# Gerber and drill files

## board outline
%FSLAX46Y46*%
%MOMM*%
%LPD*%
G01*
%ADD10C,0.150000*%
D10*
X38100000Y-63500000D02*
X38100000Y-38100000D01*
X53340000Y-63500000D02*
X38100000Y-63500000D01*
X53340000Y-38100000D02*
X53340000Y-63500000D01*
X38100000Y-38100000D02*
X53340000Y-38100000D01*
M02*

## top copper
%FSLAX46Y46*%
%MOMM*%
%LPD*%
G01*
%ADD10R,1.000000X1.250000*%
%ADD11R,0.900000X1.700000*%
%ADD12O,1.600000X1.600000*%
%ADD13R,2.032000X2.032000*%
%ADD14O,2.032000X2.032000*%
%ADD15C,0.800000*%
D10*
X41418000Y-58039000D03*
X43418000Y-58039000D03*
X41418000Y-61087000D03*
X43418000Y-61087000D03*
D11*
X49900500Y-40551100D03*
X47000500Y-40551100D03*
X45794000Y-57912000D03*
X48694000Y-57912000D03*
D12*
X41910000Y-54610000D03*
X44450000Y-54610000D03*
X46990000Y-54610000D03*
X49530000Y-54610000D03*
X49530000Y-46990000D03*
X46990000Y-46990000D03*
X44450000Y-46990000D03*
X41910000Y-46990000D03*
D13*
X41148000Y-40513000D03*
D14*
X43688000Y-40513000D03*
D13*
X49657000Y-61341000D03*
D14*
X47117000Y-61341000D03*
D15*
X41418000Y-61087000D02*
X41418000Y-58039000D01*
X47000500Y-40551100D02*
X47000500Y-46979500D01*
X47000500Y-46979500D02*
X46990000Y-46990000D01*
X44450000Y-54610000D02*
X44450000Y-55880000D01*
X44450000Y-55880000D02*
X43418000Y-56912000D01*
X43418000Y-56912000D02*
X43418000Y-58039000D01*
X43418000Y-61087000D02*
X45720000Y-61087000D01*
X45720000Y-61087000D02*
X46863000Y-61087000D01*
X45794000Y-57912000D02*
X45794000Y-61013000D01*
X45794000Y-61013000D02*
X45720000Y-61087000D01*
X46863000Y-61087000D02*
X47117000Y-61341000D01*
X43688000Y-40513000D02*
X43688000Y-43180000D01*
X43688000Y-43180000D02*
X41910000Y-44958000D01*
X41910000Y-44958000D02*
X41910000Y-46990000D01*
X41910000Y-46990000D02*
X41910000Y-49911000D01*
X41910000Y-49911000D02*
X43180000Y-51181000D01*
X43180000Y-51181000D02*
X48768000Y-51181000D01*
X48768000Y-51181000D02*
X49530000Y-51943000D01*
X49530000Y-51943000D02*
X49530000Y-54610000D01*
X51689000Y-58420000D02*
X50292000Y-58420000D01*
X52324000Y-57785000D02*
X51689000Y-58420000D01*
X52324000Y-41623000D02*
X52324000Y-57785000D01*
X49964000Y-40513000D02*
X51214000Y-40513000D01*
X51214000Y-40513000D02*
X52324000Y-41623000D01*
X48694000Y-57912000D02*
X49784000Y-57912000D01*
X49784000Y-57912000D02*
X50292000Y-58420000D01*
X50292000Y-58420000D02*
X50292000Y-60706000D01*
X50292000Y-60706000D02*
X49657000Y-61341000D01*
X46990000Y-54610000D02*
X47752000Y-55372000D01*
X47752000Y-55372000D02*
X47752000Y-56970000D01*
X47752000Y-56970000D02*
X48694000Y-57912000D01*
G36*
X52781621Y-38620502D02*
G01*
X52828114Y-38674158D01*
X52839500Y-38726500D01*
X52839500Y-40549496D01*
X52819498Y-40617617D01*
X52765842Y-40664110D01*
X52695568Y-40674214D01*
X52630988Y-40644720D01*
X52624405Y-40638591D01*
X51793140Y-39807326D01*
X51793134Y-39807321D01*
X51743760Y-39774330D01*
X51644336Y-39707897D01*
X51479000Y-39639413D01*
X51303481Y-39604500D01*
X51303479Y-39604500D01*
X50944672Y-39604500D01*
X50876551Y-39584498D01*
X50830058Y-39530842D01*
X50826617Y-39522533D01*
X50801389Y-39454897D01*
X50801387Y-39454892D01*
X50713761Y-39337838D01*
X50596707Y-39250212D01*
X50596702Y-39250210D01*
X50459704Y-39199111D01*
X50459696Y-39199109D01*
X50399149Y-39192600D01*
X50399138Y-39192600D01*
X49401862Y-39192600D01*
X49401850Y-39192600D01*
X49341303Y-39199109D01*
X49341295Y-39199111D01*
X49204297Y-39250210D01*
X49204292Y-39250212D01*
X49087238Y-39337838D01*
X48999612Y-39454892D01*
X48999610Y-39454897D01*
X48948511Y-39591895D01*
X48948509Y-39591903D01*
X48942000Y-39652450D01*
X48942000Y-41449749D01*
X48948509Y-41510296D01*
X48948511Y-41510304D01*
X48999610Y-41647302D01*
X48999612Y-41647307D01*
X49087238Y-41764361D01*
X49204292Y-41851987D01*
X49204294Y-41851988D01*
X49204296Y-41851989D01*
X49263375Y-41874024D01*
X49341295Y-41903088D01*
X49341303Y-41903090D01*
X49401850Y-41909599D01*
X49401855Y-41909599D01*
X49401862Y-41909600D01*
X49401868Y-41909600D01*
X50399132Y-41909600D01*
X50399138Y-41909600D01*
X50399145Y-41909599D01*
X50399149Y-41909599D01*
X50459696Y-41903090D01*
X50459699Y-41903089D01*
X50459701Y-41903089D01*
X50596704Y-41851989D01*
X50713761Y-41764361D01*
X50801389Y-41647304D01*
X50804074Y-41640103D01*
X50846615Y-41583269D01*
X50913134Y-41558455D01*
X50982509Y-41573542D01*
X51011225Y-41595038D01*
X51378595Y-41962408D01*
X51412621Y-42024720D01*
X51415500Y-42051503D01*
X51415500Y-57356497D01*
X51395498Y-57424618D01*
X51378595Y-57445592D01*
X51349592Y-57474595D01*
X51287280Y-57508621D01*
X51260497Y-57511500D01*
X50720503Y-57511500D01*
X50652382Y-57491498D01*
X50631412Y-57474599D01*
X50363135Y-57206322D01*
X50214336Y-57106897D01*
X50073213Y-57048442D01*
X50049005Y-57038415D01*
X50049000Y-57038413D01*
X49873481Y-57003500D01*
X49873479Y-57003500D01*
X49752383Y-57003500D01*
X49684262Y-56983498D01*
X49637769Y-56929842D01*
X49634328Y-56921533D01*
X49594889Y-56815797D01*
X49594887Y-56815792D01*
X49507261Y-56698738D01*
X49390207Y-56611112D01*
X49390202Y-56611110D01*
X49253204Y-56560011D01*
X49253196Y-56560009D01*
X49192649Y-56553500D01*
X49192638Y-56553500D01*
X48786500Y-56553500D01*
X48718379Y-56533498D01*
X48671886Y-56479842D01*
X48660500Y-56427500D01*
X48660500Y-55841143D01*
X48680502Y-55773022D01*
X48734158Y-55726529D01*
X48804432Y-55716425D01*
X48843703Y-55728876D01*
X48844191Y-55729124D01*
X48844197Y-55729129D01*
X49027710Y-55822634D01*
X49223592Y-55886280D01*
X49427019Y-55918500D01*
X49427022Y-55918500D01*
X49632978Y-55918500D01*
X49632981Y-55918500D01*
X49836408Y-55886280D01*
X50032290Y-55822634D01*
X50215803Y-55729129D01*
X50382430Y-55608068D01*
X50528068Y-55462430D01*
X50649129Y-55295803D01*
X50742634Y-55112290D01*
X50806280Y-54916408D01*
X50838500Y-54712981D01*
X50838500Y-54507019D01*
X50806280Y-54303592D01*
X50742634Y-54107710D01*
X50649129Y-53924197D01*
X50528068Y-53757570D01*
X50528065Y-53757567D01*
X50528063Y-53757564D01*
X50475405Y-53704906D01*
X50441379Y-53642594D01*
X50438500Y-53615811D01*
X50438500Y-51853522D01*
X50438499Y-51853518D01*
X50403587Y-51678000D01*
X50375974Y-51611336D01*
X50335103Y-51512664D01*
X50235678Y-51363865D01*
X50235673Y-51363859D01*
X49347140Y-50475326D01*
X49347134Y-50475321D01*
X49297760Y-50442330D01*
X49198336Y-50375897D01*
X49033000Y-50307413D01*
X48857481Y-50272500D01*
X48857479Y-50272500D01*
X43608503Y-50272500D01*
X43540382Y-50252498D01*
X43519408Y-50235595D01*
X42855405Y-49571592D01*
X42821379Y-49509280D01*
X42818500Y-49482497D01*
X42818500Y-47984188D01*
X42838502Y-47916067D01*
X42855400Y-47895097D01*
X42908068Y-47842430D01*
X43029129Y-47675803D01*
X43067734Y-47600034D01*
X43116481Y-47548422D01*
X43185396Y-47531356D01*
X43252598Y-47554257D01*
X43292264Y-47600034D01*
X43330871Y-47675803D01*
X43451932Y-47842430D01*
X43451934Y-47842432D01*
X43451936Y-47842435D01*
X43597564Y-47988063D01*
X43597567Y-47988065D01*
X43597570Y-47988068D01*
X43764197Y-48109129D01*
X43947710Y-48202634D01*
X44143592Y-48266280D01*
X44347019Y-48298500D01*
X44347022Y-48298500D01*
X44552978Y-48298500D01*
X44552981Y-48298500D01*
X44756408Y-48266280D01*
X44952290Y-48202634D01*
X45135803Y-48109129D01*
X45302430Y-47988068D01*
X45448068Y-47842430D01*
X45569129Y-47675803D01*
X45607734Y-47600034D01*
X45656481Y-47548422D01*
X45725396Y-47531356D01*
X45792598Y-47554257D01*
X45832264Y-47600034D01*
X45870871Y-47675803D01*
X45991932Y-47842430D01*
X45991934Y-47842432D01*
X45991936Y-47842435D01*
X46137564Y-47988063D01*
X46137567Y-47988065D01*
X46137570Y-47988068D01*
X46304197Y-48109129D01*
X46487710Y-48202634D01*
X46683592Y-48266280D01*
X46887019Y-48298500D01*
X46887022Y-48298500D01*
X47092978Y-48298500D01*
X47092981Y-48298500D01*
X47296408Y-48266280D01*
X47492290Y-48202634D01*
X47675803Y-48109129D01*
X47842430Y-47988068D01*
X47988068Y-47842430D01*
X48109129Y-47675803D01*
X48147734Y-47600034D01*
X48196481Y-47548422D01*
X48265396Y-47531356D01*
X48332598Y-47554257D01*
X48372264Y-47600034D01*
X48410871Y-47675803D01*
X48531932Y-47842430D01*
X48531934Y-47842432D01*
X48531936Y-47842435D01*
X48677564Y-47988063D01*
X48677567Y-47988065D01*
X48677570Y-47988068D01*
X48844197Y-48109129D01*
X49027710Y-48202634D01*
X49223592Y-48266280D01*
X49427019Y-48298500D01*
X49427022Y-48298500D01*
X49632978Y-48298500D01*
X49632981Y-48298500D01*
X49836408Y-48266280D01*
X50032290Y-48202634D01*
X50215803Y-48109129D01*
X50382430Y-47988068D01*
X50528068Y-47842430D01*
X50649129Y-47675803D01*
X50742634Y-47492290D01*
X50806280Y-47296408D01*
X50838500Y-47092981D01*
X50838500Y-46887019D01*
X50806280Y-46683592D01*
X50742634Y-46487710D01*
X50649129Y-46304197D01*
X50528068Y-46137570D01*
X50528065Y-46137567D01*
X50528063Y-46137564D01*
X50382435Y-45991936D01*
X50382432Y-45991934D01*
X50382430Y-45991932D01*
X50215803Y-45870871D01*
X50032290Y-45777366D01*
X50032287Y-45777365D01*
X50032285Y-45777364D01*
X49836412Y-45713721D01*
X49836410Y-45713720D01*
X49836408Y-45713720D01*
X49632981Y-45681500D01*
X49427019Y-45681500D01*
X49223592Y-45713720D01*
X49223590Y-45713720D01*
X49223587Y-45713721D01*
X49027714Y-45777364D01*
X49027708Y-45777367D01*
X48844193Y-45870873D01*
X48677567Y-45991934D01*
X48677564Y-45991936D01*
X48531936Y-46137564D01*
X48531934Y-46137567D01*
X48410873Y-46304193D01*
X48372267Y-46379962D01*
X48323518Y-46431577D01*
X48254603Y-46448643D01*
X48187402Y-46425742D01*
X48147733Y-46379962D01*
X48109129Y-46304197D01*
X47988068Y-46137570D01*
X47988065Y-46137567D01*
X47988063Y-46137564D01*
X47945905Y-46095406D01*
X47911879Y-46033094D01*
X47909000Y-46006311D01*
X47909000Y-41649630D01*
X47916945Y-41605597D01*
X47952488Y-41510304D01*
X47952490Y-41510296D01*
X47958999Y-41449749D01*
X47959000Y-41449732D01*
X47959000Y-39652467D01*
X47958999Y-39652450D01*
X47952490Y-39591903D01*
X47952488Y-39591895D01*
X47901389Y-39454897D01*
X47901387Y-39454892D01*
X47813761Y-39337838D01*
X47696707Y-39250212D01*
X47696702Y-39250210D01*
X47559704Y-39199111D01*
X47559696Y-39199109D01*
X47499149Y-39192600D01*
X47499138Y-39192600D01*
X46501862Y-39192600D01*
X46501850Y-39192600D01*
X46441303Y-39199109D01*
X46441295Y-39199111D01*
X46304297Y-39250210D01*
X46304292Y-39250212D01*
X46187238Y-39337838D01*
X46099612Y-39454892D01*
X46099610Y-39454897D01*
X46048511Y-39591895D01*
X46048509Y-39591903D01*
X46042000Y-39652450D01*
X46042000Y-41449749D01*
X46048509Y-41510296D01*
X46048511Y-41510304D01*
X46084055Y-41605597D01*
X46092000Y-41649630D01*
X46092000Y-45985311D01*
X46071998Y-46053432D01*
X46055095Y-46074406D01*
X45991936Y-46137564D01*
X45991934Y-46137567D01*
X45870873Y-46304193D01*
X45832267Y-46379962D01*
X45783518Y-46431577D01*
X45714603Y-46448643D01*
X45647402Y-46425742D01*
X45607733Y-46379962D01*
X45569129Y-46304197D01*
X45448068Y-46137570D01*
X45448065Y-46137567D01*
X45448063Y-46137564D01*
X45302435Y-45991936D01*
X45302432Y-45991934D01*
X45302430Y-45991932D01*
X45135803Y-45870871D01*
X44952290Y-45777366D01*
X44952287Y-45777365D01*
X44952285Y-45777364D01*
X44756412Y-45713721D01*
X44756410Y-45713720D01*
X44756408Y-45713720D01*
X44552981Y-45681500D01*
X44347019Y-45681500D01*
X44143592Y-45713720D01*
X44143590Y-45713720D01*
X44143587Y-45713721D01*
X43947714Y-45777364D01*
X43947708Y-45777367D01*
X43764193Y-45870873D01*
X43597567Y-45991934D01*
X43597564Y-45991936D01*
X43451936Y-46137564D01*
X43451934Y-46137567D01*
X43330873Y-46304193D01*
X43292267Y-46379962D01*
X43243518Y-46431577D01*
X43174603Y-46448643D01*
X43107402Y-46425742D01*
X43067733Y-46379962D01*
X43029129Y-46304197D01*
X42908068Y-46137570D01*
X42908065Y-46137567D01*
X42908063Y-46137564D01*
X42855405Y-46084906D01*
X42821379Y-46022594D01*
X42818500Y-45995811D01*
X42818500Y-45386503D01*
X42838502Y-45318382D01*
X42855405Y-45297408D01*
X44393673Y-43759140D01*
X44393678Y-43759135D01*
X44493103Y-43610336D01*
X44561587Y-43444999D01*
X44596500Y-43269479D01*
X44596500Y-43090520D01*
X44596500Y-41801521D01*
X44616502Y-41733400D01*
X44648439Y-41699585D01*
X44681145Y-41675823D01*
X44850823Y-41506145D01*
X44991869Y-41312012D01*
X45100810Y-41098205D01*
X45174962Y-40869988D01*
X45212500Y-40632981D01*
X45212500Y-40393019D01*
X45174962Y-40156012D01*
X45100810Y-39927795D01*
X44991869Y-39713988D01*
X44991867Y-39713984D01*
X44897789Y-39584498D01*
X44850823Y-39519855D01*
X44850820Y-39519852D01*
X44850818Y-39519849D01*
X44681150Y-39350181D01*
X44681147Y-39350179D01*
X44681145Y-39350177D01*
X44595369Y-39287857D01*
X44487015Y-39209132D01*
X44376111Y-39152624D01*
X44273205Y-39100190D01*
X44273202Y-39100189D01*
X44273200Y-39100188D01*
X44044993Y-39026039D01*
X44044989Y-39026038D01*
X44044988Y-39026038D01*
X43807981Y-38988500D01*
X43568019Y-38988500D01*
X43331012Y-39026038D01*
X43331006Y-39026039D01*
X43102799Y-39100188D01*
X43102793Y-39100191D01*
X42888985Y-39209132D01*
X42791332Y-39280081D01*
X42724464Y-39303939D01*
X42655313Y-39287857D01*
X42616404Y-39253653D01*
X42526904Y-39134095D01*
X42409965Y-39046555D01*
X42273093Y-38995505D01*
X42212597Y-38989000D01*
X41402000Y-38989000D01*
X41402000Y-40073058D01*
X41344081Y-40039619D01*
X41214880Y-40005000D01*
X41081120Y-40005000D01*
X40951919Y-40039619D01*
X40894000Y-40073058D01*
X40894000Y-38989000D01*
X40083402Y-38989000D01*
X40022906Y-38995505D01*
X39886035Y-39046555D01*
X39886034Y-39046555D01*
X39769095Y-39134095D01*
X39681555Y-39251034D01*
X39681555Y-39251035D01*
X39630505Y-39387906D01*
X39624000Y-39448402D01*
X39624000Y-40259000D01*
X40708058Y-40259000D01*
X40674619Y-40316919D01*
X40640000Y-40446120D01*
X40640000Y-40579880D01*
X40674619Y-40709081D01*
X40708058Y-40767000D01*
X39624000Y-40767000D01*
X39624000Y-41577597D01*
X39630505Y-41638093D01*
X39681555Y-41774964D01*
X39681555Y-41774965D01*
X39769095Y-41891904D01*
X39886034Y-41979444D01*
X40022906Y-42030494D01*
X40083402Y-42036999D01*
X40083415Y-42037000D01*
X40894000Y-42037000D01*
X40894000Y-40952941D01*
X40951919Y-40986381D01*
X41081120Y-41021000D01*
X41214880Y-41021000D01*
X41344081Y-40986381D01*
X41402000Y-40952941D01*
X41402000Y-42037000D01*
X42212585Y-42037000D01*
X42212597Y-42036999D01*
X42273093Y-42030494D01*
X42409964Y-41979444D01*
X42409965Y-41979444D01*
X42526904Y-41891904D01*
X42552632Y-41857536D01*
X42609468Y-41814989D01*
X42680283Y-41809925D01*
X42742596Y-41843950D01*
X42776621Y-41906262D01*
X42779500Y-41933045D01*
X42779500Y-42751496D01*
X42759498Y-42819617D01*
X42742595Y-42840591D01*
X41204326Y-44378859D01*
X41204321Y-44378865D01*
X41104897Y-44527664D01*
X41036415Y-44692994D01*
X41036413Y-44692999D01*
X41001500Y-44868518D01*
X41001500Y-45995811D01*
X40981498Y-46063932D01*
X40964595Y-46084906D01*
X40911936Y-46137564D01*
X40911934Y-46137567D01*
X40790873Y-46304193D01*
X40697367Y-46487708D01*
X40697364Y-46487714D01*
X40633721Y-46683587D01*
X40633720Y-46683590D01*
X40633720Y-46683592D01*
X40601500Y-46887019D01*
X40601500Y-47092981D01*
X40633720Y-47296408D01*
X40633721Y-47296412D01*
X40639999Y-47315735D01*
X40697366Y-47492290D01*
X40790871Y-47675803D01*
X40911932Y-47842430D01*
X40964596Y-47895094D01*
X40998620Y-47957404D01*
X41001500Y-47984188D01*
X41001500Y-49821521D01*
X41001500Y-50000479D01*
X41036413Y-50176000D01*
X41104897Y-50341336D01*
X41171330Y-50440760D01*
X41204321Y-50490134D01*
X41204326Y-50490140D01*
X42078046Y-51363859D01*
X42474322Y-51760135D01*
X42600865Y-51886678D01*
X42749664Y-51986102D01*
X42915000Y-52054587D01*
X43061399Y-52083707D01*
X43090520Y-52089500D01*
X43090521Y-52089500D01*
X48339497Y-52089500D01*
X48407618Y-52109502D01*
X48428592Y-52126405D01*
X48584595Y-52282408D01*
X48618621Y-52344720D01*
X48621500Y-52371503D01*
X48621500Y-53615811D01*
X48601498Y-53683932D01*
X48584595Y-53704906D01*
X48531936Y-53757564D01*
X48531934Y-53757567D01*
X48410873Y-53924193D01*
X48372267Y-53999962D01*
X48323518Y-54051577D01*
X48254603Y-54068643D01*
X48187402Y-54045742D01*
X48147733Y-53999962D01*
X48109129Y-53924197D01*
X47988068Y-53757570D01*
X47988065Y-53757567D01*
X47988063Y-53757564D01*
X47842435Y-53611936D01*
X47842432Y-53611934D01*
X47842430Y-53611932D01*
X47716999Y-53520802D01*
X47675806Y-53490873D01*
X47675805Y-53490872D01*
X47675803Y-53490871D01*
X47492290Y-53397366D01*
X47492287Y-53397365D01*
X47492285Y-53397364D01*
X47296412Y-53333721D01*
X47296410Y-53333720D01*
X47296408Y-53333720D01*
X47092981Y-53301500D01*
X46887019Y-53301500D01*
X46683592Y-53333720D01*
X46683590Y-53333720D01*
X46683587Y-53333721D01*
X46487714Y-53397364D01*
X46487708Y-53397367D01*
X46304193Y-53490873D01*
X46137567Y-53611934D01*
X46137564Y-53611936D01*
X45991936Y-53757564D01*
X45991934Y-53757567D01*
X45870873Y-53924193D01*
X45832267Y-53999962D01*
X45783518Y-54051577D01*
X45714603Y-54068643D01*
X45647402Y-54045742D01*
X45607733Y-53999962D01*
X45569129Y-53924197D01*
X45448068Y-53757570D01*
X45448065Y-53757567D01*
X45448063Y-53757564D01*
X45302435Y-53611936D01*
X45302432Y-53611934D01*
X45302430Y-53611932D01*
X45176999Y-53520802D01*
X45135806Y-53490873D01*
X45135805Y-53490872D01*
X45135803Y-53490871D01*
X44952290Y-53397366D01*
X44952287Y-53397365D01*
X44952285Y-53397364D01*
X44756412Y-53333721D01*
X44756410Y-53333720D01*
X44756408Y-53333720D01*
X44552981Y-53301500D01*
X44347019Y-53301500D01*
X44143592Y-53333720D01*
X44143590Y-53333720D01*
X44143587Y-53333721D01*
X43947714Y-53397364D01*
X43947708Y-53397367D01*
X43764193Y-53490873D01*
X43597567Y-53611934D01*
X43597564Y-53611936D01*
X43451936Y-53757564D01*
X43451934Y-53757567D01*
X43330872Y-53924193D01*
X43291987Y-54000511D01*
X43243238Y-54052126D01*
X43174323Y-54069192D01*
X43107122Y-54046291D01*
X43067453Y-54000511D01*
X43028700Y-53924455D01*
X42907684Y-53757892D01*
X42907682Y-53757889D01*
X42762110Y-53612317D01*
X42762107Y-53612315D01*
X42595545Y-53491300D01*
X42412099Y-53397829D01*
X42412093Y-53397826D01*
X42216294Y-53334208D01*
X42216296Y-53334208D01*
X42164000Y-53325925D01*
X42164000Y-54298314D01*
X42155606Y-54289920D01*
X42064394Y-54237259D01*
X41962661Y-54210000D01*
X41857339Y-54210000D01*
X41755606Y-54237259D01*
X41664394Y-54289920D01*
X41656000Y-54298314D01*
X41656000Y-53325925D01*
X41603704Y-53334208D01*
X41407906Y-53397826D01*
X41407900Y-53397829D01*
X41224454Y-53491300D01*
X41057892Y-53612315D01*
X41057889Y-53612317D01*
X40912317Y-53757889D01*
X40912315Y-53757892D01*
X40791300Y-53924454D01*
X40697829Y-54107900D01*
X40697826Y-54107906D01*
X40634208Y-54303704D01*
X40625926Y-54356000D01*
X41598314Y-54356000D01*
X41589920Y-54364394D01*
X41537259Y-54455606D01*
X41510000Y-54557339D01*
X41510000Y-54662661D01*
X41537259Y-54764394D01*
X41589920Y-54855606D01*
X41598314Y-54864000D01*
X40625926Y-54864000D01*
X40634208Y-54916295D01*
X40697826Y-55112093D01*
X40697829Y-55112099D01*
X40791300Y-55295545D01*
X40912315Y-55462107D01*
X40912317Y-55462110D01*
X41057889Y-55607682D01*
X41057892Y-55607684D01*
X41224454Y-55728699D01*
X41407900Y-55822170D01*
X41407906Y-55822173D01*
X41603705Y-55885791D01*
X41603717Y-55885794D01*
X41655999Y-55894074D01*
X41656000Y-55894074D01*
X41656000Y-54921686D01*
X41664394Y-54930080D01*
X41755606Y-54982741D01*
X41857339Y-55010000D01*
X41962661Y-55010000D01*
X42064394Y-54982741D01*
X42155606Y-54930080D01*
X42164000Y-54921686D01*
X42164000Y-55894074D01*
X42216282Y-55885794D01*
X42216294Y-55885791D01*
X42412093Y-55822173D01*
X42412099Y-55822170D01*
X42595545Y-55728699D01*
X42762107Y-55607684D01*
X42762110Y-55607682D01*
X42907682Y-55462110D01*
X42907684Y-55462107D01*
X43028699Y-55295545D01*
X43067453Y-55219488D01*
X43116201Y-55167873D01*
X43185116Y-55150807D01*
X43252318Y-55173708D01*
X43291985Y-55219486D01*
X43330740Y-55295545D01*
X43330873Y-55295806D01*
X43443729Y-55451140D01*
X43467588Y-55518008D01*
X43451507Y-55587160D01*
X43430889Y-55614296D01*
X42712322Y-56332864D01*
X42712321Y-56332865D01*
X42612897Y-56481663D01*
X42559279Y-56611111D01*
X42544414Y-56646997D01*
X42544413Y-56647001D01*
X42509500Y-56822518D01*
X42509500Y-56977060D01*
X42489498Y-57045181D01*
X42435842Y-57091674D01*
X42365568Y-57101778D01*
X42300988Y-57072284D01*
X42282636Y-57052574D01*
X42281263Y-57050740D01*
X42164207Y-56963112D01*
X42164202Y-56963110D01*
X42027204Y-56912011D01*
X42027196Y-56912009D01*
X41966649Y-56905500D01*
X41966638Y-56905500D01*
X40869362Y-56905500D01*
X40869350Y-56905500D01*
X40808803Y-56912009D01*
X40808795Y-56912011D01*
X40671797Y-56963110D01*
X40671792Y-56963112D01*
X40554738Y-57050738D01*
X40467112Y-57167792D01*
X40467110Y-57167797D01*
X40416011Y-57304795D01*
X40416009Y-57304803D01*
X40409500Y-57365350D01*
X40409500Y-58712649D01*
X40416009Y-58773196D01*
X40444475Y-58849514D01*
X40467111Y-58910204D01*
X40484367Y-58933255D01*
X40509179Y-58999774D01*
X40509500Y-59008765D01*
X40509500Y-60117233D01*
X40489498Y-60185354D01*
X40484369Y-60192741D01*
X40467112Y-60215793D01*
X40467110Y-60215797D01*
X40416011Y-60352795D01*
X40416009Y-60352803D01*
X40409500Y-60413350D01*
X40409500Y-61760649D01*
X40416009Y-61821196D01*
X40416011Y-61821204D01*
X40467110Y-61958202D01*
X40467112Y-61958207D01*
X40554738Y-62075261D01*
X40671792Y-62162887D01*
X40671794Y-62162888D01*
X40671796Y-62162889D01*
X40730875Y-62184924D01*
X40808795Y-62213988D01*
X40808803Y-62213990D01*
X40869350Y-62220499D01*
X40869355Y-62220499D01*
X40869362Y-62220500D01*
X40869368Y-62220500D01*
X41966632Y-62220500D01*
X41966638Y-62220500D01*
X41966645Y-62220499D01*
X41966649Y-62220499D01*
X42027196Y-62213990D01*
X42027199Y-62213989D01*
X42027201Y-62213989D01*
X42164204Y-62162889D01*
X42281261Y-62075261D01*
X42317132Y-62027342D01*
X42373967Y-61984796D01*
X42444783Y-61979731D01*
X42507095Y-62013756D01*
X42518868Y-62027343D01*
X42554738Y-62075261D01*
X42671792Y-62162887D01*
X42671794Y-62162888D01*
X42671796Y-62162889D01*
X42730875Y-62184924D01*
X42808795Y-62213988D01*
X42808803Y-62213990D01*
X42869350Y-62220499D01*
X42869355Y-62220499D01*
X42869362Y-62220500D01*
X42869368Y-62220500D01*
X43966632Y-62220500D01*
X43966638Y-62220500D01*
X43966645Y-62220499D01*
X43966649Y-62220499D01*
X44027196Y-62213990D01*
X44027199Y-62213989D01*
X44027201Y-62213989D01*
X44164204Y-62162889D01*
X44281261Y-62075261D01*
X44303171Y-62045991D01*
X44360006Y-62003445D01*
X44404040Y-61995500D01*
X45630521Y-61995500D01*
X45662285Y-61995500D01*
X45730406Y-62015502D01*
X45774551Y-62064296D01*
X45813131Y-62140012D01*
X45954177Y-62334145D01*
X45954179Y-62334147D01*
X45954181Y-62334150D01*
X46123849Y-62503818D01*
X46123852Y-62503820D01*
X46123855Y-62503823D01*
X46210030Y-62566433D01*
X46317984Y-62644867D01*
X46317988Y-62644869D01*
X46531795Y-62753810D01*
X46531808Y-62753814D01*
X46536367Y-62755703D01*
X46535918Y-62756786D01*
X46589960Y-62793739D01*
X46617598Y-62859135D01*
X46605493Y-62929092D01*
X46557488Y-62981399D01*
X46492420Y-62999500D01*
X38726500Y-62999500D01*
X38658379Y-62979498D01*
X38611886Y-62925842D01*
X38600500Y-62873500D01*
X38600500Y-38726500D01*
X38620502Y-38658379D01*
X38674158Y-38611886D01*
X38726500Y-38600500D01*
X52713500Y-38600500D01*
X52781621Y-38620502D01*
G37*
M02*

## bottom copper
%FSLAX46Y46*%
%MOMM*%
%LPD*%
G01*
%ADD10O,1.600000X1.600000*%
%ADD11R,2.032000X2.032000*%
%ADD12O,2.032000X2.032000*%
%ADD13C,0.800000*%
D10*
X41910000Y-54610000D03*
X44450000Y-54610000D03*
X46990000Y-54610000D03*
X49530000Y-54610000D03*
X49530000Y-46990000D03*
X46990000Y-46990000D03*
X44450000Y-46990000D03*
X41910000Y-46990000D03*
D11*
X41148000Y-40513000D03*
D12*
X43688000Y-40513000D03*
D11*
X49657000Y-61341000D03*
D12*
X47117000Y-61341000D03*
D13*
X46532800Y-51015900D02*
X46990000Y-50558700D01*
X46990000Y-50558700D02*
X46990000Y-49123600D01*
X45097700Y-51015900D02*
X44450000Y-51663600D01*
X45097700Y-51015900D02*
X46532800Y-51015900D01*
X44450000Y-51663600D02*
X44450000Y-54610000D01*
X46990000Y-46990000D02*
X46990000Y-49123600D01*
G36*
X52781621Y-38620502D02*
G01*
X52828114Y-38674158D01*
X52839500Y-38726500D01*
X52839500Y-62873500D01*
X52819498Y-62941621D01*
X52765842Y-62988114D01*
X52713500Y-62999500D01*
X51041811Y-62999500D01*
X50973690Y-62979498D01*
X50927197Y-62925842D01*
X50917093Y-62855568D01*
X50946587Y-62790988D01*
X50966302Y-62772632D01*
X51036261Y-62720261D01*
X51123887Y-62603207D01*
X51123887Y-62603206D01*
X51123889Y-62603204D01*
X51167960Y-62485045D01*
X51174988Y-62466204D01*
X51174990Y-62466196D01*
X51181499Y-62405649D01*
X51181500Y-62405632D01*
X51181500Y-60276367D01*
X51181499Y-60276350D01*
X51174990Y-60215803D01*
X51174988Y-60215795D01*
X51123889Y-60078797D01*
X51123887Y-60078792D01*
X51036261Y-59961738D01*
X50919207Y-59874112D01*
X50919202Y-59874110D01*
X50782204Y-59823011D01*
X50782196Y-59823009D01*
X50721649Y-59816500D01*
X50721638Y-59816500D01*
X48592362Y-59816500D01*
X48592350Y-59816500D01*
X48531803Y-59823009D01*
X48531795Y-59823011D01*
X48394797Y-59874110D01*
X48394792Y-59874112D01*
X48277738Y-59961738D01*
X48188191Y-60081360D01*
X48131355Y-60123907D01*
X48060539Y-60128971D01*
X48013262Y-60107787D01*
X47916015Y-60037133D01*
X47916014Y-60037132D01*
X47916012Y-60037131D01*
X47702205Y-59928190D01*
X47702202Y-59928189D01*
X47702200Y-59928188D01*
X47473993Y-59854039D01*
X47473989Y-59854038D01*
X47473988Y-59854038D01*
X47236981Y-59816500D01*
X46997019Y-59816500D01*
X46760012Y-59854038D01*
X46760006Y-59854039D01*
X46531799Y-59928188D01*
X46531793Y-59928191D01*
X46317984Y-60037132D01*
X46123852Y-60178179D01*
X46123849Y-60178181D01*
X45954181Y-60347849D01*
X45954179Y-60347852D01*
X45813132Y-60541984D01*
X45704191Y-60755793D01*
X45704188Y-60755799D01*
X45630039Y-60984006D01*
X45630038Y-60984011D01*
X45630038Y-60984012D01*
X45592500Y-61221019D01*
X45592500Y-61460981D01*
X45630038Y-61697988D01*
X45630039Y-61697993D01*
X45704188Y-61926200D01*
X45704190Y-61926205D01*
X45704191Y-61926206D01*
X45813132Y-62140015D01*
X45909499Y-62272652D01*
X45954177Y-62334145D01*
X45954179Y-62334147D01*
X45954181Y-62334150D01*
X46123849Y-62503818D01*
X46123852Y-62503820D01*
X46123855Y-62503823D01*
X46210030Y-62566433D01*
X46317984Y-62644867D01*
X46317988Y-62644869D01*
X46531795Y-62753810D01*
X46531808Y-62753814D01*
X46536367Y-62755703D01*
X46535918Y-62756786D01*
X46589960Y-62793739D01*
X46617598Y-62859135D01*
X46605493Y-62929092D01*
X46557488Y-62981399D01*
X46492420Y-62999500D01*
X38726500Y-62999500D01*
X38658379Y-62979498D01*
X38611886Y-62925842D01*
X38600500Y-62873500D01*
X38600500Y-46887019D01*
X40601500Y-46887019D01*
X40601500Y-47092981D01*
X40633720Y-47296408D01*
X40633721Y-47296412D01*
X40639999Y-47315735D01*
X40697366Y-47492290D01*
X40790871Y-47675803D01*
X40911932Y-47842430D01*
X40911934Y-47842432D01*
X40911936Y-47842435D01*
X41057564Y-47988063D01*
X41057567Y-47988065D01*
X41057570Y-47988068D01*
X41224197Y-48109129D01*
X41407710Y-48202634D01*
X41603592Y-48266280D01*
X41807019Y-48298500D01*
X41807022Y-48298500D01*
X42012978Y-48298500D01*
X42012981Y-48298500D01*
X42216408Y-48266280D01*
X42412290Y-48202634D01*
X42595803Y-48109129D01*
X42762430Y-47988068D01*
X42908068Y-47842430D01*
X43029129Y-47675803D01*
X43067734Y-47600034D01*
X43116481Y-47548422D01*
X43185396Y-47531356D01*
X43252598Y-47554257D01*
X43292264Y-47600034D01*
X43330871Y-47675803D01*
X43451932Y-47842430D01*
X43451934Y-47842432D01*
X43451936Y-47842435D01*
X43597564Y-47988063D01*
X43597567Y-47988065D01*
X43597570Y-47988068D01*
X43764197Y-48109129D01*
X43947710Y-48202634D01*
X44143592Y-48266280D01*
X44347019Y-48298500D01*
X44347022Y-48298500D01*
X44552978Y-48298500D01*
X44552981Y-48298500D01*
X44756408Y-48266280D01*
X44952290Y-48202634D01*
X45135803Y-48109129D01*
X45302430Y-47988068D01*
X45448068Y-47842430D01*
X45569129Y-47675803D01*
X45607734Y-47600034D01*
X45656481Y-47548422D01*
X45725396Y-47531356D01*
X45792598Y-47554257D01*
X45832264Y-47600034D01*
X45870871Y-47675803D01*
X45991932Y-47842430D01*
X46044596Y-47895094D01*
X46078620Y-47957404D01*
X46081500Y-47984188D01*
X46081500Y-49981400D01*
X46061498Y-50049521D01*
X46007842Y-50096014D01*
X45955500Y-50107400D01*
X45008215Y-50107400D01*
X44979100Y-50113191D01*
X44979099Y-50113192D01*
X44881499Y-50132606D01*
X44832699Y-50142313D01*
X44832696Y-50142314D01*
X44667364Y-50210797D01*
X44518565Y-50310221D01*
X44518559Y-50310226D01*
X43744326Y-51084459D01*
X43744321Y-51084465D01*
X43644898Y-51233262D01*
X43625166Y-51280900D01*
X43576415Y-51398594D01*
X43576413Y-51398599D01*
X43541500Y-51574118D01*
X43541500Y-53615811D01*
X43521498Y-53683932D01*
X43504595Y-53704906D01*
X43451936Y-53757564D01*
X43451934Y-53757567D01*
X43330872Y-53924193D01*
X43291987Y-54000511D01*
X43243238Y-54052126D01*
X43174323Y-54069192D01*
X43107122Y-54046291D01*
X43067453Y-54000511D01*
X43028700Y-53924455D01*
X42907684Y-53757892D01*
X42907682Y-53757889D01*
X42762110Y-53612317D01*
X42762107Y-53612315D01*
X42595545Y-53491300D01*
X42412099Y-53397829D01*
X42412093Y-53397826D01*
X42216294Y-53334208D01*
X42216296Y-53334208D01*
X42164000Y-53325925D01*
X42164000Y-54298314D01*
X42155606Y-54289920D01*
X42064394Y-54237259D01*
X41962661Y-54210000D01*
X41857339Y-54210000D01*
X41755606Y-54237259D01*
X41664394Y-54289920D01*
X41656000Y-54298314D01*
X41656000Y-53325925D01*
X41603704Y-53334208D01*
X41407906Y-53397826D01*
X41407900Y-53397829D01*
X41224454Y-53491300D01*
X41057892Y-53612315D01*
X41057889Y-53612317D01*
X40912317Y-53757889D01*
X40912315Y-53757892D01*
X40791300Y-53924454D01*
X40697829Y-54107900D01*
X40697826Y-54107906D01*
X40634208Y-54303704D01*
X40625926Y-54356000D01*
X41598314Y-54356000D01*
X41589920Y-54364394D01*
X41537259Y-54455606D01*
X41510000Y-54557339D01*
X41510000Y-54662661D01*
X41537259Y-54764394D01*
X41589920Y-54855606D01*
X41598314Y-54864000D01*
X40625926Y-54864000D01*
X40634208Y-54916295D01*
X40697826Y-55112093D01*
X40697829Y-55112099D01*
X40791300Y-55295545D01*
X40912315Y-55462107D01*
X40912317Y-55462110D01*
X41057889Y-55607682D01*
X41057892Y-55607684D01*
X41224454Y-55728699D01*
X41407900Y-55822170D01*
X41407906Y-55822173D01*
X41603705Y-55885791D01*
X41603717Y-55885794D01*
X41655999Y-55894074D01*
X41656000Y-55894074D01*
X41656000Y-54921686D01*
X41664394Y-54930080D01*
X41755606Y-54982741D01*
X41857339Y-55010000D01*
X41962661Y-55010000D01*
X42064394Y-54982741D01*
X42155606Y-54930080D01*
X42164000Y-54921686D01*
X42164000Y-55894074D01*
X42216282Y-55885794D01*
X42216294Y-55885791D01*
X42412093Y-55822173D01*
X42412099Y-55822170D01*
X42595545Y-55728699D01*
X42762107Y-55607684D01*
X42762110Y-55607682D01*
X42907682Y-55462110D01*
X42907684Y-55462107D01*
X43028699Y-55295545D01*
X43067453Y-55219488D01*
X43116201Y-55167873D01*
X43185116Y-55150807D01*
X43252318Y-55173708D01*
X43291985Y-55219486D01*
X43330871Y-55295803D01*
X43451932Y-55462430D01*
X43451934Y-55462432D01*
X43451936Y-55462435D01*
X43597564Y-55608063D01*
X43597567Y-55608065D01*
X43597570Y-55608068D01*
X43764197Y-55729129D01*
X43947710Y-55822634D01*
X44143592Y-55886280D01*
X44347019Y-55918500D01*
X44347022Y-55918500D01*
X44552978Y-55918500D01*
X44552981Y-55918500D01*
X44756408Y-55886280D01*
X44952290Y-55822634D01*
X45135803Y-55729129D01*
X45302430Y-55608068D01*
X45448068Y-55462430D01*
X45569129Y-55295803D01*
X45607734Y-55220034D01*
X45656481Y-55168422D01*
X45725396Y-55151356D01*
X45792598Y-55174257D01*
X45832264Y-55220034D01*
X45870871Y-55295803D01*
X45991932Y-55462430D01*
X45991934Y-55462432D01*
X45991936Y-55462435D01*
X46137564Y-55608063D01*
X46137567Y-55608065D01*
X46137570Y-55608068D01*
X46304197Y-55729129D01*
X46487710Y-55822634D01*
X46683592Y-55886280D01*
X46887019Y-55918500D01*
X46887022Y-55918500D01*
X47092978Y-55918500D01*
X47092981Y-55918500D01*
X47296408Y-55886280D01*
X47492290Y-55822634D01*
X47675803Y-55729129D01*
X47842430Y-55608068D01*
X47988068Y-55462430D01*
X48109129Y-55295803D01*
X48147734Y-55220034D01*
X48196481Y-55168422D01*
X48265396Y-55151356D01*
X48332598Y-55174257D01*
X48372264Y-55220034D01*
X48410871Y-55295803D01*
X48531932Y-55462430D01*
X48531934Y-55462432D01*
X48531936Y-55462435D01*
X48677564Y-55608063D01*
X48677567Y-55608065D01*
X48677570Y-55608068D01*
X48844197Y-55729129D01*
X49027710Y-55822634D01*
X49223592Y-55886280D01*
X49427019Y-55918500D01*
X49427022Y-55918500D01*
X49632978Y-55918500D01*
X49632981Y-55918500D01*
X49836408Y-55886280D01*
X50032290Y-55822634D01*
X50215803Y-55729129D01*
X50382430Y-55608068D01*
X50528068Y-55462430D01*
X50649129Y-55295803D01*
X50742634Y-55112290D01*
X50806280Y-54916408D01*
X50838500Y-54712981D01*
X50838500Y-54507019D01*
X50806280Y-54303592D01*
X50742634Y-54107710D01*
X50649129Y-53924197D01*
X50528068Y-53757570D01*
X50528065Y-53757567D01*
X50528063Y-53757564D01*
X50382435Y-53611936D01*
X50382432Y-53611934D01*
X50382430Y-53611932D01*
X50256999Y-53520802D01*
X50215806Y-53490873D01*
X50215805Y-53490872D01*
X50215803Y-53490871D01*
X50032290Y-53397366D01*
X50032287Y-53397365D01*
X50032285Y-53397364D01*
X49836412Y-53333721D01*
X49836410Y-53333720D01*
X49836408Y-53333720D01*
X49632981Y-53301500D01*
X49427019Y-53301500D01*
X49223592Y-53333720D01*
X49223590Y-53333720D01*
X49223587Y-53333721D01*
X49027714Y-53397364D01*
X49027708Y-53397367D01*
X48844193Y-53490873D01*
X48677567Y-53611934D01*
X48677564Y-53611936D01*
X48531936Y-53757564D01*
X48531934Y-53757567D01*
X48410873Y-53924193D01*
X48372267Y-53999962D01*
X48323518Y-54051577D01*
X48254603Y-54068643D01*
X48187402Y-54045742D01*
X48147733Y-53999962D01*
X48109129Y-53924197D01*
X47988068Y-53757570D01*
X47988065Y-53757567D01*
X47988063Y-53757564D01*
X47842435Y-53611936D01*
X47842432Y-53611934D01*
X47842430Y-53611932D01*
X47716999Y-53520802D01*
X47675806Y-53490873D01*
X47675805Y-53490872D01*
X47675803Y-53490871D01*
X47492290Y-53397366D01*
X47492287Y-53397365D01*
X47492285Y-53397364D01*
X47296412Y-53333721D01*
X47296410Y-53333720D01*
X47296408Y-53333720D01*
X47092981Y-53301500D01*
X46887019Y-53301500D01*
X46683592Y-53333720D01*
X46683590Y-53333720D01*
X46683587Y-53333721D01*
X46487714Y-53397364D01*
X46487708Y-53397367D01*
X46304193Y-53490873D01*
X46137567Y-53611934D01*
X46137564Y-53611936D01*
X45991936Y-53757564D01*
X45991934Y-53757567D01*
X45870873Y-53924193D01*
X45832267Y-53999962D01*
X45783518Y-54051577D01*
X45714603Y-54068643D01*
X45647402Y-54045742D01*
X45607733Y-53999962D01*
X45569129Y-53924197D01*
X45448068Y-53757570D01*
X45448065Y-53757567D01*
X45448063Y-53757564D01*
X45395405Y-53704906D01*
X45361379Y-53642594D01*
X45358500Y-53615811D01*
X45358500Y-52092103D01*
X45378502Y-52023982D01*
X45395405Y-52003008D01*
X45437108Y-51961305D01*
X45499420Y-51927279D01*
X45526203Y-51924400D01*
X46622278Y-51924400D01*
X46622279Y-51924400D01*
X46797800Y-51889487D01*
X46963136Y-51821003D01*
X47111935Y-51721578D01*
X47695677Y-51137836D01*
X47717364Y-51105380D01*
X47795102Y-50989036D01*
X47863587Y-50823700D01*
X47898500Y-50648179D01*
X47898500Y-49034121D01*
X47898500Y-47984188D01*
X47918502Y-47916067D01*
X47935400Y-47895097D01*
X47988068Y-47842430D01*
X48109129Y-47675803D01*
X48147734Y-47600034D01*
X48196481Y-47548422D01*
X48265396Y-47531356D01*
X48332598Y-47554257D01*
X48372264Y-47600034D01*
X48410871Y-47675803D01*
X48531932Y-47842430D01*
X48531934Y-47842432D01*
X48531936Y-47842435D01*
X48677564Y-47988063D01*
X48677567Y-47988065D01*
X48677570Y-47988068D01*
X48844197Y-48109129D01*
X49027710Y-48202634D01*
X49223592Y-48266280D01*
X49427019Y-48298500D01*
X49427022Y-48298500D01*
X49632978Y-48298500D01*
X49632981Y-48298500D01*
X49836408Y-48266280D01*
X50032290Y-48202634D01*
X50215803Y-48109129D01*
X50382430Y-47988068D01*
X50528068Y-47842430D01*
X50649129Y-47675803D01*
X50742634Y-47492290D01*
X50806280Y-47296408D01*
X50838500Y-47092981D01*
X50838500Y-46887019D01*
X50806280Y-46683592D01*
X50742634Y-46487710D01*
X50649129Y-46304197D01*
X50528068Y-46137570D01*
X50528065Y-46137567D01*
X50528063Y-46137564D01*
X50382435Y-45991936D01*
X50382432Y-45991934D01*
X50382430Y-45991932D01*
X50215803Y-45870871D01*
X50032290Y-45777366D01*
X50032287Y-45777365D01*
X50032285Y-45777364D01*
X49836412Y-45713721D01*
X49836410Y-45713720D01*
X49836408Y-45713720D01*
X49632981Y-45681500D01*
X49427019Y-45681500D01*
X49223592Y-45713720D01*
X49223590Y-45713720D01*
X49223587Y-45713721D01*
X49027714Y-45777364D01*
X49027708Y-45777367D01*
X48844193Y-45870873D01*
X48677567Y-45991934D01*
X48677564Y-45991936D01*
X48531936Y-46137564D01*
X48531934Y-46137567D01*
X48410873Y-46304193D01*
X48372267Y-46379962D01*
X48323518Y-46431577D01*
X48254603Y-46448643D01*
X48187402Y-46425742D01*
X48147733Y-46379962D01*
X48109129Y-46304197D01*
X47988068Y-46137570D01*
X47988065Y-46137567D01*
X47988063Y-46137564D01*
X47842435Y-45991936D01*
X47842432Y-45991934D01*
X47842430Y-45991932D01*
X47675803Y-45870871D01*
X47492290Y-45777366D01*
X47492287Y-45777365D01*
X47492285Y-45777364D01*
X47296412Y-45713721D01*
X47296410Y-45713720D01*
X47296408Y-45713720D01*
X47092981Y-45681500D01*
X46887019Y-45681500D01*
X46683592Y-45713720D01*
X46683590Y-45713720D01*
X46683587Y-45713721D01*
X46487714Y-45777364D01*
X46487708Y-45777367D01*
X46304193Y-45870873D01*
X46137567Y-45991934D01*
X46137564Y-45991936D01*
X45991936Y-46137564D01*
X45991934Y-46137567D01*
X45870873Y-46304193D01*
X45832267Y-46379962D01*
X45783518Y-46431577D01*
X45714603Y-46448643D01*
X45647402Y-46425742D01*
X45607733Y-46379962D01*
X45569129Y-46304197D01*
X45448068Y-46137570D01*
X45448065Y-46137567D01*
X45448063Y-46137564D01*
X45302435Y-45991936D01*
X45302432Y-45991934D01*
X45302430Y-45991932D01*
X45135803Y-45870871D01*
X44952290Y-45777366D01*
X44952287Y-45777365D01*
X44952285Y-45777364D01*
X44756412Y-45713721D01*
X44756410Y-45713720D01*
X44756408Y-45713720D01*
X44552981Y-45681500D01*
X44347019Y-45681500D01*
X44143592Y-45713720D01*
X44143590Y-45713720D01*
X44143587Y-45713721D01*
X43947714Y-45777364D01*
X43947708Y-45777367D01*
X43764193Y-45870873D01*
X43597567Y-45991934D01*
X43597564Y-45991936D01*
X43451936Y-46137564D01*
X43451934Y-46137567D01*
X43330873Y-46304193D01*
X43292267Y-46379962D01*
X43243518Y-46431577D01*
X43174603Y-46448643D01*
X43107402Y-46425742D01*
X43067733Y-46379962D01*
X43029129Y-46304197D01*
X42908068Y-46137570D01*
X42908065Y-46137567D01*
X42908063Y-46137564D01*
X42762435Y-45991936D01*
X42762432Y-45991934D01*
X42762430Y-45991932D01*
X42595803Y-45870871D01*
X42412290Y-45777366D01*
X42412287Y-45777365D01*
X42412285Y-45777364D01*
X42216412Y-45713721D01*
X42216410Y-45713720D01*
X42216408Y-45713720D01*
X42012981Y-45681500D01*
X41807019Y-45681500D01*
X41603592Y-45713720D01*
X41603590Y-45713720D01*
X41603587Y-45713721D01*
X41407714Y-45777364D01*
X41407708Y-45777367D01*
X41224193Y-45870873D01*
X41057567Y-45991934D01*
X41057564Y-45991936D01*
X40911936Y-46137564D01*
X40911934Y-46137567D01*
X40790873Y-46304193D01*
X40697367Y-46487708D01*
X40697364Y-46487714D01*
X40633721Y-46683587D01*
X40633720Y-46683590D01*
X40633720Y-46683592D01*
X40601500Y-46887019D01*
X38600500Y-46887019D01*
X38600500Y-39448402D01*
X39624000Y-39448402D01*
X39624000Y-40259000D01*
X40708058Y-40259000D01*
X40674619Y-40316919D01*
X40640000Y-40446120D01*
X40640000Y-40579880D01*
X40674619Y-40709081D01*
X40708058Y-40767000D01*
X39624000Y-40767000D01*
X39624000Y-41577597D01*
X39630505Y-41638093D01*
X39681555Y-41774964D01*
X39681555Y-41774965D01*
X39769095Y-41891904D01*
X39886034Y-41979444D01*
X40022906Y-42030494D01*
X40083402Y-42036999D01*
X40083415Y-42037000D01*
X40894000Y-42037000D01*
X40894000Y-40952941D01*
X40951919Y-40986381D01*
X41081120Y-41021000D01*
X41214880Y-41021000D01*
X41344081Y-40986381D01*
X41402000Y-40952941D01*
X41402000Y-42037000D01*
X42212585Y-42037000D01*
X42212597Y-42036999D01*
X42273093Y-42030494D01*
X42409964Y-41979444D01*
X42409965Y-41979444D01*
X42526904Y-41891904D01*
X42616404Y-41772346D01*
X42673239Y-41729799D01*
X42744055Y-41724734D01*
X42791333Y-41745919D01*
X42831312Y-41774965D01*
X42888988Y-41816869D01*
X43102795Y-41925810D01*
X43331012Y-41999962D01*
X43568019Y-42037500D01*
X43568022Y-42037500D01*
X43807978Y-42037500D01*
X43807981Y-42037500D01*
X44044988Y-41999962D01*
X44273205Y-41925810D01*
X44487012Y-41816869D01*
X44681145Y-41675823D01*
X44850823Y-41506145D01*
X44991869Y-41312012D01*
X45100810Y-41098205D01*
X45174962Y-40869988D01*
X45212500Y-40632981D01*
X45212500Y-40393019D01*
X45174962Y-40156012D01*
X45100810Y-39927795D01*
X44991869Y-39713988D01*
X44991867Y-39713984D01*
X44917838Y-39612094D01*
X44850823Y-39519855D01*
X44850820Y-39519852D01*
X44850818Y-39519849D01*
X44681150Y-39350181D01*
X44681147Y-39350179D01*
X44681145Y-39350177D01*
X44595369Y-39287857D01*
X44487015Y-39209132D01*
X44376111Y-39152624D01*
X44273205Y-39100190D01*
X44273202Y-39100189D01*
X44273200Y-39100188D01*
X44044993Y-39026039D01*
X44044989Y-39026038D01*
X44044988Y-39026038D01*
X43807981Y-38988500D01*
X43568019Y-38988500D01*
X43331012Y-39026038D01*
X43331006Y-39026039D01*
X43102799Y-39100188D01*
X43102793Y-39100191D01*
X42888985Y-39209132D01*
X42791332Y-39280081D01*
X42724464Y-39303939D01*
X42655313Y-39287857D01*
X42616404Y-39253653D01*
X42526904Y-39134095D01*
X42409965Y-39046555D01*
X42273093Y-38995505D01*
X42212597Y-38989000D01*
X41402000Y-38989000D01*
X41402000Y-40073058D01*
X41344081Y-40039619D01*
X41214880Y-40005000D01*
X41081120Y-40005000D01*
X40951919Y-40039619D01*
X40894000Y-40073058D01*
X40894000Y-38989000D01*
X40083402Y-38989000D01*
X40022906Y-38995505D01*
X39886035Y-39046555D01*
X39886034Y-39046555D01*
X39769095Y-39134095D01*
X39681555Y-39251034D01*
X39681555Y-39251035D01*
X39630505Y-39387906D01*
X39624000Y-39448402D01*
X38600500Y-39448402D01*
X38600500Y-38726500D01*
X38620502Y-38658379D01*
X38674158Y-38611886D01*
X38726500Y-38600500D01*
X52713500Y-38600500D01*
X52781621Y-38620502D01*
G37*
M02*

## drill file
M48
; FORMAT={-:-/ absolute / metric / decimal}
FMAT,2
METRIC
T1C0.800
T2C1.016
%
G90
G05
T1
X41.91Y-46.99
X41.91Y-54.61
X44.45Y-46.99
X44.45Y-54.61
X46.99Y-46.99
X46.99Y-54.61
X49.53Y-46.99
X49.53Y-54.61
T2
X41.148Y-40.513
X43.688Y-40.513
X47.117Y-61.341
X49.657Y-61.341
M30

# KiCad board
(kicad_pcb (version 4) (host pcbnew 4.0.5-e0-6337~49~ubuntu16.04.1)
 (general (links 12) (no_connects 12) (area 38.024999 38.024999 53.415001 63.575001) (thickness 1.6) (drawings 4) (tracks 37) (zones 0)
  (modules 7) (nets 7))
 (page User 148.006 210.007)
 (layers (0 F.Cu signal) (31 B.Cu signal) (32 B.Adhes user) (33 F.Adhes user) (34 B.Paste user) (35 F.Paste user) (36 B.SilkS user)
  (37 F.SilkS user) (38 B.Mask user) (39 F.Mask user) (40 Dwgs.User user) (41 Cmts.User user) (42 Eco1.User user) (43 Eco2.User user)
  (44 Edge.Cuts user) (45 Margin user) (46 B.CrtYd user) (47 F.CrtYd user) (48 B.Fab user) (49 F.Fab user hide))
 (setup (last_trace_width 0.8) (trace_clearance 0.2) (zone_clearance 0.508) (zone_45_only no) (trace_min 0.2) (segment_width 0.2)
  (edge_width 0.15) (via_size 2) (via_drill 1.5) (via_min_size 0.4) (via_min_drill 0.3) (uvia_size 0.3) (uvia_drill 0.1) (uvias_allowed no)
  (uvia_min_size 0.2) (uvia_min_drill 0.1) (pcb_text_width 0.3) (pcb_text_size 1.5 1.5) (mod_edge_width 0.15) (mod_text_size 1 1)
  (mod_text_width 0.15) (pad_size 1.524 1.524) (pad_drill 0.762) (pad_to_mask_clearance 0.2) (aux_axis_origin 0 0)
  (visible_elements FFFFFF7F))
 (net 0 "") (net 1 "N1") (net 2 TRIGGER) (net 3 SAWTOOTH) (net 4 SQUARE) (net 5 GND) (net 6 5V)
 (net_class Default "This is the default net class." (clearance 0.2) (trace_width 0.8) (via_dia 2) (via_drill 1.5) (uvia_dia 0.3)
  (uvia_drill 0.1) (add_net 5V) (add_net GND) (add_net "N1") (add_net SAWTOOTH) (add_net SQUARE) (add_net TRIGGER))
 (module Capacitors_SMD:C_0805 (layer F.Cu) (at 42.418 58.039)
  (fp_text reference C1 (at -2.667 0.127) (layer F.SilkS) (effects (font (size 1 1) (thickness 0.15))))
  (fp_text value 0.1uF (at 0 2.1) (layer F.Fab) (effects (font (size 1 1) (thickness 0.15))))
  (pad 1 smd rect (at -1 0) (size 1 1.25) (layers F.Cu F.Paste F.Mask) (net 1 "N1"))
  (pad 2 smd rect (at 1 0) (size 1 1.25) (layers F.Cu F.Paste F.Mask) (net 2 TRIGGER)))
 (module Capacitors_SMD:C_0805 (layer F.Cu) (at 42.418 61.087)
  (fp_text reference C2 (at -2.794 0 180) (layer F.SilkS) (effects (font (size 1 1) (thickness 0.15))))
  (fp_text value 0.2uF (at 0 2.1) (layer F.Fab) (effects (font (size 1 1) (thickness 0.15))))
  (pad 1 smd rect (at -1 0) (size 1 1.25) (layers F.Cu F.Paste F.Mask) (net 1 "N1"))
  (pad 2 smd rect (at 1 0) (size 1 1.25) (layers F.Cu F.Paste F.Mask) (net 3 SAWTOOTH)))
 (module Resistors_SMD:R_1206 (layer F.Cu) (at 48.4505 40.5511 180)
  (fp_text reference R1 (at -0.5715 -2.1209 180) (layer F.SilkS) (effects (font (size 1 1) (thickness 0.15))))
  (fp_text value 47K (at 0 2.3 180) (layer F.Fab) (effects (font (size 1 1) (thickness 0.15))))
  (pad 1 smd rect (at -1.45 0 180) (size 0.9 1.7) (layers F.Cu F.Paste F.Mask) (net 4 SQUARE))
  (pad 2 smd rect (at 1.45 0 180) (size 0.9 1.7) (layers F.Cu F.Paste F.Mask) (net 2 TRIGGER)))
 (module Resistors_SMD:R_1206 (layer F.Cu) (at 47.244 57.912)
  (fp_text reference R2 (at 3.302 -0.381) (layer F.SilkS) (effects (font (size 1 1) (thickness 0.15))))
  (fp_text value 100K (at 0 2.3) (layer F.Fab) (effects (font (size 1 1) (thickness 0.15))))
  (pad 1 smd rect (at -1.45 0) (size 0.9 1.7) (layers F.Cu F.Paste F.Mask) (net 3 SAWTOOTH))
  (pad 2 smd rect (at 1.45 0) (size 0.9 1.7) (layers F.Cu F.Paste F.Mask) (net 4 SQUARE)))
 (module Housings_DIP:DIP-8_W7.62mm (layer F.Cu) (at 41.91 54.61 90)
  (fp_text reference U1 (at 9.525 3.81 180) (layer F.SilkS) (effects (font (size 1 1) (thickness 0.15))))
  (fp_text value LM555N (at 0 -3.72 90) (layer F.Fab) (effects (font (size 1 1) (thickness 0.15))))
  (pad 1 thru_hole oval (at 0 0 90) (size 1.6 1.6) (drill 0.8) (layers *.Cu *.Mask F.SilkS) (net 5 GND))
  (pad 2 thru_hole oval (at 0 2.54 90) (size 1.6 1.6) (drill 0.8) (layers *.Cu *.Mask F.SilkS) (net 2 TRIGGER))
  (pad 3 thru_hole oval (at 0 5.08 90) (size 1.6 1.6) (drill 0.8) (layers *.Cu *.Mask F.SilkS) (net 4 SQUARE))
  (pad 4 thru_hole oval (at 0 7.62 90) (size 1.6 1.6) (drill 0.8) (layers *.Cu *.Mask F.SilkS) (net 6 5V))
  (pad 5 thru_hole oval (at 7.62 7.62 90) (size 1.6 1.6) (drill 0.8) (layers *.Cu *.Mask F.SilkS))
  (pad 6 thru_hole oval (at 7.62 5.08 90) (size 1.6 1.6) (drill 0.8) (layers *.Cu *.Mask F.SilkS) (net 2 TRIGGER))
  (pad 7 thru_hole oval (at 7.62 2.54 90) (size 1.6 1.6) (drill 0.8) (layers *.Cu *.Mask F.SilkS))
  (pad 8 thru_hole oval (at 7.62 0 90) (size 1.6 1.6) (drill 0.8) (layers *.Cu *.Mask F.SilkS) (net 6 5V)))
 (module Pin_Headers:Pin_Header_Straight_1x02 (layer F.Cu) (at 41.148 40.513 90)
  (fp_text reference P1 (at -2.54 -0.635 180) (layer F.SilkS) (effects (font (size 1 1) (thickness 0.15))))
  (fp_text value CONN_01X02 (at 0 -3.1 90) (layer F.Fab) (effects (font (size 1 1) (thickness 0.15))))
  (pad 1 thru_hole rect (at 0 0 90) (size 2.032 2.032) (drill 1.016) (layers *.Cu *.Mask F.SilkS) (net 5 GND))
  (pad 2 thru_hole oval (at 0 2.54 90) (size 2.032 2.032) (drill 1.016) (layers *.Cu *.Mask F.SilkS) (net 6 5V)))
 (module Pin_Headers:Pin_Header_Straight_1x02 (layer F.Cu) (at 49.657 61.341 270)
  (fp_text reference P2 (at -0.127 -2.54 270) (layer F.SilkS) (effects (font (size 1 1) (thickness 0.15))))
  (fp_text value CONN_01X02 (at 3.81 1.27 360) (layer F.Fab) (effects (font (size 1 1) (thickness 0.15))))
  (pad 1 thru_hole rect (at 0 0 270) (size 2.032 2.032) (drill 1.016) (layers *.Cu *.Mask F.SilkS) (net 4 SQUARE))
  (pad 2 thru_hole oval (at 0 2.54 270) (size 2.032 2.032) (drill 1.016) (layers *.Cu *.Mask F.SilkS) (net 3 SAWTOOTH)))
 (gr_line (start 38.1 63.5) (end 38.1 38.1) (layer Edge.Cuts) (width 0.15))
 (gr_line (start 53.34 63.5) (end 38.1 63.5) (layer Edge.Cuts) (width 0.15))
 (gr_line (start 53.34 38.1) (end 53.34 63.5) (layer Edge.Cuts) (width 0.15))
 (gr_line (start 38.1 38.1) (end 53.34 38.1) (layer Edge.Cuts) (width 0.15))
 (segment (start 41.418 61.087) (end 41.418 58.039) (width 0.8) (layer F.Cu) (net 1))
 (segment (start 46.5328 51.0159) (end 46.99 50.5587) (width 0.8) (layer B.Cu) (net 2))
 (segment (start 46.99 50.5587) (end 46.99 49.1236) (width 0.8) (layer B.Cu) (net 2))
 (segment (start 45.0977 51.0159) (end 44.45 51.6636) (width 0.8) (layer B.Cu) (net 2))
 (segment (start 45.0977 51.0159) (end 46.5328 51.0159) (width 0.8) (layer B.Cu) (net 2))
 (segment (start 44.45 51.6636) (end 44.45 54.61) (width 0.8) (layer B.Cu) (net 2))
 (segment (start 46.99 46.99) (end 46.99 49.1236) (width 0.8) (layer B.Cu) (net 2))
 (segment (start 47.0005 40.5511) (end 47.0005 46.9795) (width 0.8) (layer F.Cu) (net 2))
 (segment (start 47.0005 46.9795) (end 46.99 46.99) (width 0.8) (layer F.Cu) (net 2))
 (segment (start 44.45 54.61) (end 44.45 55.88) (width 0.8) (layer F.Cu) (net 2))
 (segment (start 44.45 55.88) (end 43.418 56.912) (width 0.8) (layer F.Cu) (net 2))
 (segment (start 43.418 56.912) (end 43.418 58.039) (width 0.8) (layer F.Cu) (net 2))
 (segment (start 43.418 61.087) (end 45.72 61.087) (width 0.8) (layer F.Cu) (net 3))
 (segment (start 45.72 61.087) (end 46.863 61.087) (width 0.8) (layer F.Cu) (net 3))
 (segment (start 45.794 57.912) (end 45.794 61.013) (width 0.8) (layer F.Cu) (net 3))
 (segment (start 45.794 61.013) (end 45.72 61.087) (width 0.8) (layer F.Cu) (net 3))
 (segment (start 46.863 61.087) (end 47.117 61.341) (width 0.8) (layer F.Cu) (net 3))
 (segment (start 43.688 40.513) (end 43.688 43.18) (width 0.8) (layer F.Cu) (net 6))
 (segment (start 43.688 43.18) (end 41.91 44.958) (width 0.8) (layer F.Cu) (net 6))
 (segment (start 41.91 44.958) (end 41.91 46.99) (width 0.8) (layer F.Cu) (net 6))
 (segment (start 41.91 46.99) (end 41.91 49.911) (width 0.8) (layer F.Cu) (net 6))
 (segment (start 41.91 49.911) (end 43.18 51.181) (width 0.8) (layer F.Cu) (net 6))
 (segment (start 43.18 51.181) (end 48.768 51.181) (width 0.8) (layer F.Cu) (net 6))
 (segment (start 48.768 51.181) (end 49.53 51.943) (width 0.8) (layer F.Cu) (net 6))
 (segment (start 49.53 51.943) (end 49.53 54.61) (width 0.8) (layer F.Cu) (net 6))
 (segment (start 51.689 58.42) (end 50.292 58.42) (width 0.8) (layer F.Cu) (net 4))
 (segment (start 52.324 57.785) (end 51.689 58.42) (width 0.8) (layer F.Cu) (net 4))
 (segment (start 52.324 41.623) (end 52.324 57.785) (width 0.8) (layer F.Cu) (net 4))
 (segment (start 49.964 40.513) (end 51.214 40.513) (width 0.8) (layer F.Cu) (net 4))
 (segment (start 51.214 40.513) (end 52.324 41.623) (width 0.8) (layer F.Cu) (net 4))
 (segment (start 48.694 57.912) (end 49.784 57.912) (width 0.8) (layer F.Cu) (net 4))
 (segment (start 49.784 57.912) (end 50.292 58.42) (width 0.8) (layer F.Cu) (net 4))
 (segment (start 50.292 58.42) (end 50.292 60.706) (width 0.8) (layer F.Cu) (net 4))
 (segment (start 50.292 60.706) (end 49.657 61.341) (width 0.8) (layer F.Cu) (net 4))
 (segment (start 46.99 54.61) (end 47.752 55.372) (width 0.8) (layer F.Cu) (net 4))
 (segment (start 47.752 55.372) (end 47.752 56.97) (width 0.8) (layer F.Cu) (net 4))
 (segment (start 47.752 56.97) (end 48.694 57.912) (width 0.8) (layer F.Cu) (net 4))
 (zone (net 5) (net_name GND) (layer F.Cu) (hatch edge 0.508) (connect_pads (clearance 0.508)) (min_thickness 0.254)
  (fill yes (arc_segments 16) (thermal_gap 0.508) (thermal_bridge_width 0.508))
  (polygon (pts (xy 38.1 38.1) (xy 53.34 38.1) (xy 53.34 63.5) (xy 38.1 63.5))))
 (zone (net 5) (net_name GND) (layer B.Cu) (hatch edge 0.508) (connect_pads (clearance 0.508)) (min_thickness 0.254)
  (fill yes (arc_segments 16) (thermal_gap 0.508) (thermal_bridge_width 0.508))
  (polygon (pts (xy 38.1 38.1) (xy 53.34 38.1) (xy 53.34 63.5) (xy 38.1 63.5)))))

